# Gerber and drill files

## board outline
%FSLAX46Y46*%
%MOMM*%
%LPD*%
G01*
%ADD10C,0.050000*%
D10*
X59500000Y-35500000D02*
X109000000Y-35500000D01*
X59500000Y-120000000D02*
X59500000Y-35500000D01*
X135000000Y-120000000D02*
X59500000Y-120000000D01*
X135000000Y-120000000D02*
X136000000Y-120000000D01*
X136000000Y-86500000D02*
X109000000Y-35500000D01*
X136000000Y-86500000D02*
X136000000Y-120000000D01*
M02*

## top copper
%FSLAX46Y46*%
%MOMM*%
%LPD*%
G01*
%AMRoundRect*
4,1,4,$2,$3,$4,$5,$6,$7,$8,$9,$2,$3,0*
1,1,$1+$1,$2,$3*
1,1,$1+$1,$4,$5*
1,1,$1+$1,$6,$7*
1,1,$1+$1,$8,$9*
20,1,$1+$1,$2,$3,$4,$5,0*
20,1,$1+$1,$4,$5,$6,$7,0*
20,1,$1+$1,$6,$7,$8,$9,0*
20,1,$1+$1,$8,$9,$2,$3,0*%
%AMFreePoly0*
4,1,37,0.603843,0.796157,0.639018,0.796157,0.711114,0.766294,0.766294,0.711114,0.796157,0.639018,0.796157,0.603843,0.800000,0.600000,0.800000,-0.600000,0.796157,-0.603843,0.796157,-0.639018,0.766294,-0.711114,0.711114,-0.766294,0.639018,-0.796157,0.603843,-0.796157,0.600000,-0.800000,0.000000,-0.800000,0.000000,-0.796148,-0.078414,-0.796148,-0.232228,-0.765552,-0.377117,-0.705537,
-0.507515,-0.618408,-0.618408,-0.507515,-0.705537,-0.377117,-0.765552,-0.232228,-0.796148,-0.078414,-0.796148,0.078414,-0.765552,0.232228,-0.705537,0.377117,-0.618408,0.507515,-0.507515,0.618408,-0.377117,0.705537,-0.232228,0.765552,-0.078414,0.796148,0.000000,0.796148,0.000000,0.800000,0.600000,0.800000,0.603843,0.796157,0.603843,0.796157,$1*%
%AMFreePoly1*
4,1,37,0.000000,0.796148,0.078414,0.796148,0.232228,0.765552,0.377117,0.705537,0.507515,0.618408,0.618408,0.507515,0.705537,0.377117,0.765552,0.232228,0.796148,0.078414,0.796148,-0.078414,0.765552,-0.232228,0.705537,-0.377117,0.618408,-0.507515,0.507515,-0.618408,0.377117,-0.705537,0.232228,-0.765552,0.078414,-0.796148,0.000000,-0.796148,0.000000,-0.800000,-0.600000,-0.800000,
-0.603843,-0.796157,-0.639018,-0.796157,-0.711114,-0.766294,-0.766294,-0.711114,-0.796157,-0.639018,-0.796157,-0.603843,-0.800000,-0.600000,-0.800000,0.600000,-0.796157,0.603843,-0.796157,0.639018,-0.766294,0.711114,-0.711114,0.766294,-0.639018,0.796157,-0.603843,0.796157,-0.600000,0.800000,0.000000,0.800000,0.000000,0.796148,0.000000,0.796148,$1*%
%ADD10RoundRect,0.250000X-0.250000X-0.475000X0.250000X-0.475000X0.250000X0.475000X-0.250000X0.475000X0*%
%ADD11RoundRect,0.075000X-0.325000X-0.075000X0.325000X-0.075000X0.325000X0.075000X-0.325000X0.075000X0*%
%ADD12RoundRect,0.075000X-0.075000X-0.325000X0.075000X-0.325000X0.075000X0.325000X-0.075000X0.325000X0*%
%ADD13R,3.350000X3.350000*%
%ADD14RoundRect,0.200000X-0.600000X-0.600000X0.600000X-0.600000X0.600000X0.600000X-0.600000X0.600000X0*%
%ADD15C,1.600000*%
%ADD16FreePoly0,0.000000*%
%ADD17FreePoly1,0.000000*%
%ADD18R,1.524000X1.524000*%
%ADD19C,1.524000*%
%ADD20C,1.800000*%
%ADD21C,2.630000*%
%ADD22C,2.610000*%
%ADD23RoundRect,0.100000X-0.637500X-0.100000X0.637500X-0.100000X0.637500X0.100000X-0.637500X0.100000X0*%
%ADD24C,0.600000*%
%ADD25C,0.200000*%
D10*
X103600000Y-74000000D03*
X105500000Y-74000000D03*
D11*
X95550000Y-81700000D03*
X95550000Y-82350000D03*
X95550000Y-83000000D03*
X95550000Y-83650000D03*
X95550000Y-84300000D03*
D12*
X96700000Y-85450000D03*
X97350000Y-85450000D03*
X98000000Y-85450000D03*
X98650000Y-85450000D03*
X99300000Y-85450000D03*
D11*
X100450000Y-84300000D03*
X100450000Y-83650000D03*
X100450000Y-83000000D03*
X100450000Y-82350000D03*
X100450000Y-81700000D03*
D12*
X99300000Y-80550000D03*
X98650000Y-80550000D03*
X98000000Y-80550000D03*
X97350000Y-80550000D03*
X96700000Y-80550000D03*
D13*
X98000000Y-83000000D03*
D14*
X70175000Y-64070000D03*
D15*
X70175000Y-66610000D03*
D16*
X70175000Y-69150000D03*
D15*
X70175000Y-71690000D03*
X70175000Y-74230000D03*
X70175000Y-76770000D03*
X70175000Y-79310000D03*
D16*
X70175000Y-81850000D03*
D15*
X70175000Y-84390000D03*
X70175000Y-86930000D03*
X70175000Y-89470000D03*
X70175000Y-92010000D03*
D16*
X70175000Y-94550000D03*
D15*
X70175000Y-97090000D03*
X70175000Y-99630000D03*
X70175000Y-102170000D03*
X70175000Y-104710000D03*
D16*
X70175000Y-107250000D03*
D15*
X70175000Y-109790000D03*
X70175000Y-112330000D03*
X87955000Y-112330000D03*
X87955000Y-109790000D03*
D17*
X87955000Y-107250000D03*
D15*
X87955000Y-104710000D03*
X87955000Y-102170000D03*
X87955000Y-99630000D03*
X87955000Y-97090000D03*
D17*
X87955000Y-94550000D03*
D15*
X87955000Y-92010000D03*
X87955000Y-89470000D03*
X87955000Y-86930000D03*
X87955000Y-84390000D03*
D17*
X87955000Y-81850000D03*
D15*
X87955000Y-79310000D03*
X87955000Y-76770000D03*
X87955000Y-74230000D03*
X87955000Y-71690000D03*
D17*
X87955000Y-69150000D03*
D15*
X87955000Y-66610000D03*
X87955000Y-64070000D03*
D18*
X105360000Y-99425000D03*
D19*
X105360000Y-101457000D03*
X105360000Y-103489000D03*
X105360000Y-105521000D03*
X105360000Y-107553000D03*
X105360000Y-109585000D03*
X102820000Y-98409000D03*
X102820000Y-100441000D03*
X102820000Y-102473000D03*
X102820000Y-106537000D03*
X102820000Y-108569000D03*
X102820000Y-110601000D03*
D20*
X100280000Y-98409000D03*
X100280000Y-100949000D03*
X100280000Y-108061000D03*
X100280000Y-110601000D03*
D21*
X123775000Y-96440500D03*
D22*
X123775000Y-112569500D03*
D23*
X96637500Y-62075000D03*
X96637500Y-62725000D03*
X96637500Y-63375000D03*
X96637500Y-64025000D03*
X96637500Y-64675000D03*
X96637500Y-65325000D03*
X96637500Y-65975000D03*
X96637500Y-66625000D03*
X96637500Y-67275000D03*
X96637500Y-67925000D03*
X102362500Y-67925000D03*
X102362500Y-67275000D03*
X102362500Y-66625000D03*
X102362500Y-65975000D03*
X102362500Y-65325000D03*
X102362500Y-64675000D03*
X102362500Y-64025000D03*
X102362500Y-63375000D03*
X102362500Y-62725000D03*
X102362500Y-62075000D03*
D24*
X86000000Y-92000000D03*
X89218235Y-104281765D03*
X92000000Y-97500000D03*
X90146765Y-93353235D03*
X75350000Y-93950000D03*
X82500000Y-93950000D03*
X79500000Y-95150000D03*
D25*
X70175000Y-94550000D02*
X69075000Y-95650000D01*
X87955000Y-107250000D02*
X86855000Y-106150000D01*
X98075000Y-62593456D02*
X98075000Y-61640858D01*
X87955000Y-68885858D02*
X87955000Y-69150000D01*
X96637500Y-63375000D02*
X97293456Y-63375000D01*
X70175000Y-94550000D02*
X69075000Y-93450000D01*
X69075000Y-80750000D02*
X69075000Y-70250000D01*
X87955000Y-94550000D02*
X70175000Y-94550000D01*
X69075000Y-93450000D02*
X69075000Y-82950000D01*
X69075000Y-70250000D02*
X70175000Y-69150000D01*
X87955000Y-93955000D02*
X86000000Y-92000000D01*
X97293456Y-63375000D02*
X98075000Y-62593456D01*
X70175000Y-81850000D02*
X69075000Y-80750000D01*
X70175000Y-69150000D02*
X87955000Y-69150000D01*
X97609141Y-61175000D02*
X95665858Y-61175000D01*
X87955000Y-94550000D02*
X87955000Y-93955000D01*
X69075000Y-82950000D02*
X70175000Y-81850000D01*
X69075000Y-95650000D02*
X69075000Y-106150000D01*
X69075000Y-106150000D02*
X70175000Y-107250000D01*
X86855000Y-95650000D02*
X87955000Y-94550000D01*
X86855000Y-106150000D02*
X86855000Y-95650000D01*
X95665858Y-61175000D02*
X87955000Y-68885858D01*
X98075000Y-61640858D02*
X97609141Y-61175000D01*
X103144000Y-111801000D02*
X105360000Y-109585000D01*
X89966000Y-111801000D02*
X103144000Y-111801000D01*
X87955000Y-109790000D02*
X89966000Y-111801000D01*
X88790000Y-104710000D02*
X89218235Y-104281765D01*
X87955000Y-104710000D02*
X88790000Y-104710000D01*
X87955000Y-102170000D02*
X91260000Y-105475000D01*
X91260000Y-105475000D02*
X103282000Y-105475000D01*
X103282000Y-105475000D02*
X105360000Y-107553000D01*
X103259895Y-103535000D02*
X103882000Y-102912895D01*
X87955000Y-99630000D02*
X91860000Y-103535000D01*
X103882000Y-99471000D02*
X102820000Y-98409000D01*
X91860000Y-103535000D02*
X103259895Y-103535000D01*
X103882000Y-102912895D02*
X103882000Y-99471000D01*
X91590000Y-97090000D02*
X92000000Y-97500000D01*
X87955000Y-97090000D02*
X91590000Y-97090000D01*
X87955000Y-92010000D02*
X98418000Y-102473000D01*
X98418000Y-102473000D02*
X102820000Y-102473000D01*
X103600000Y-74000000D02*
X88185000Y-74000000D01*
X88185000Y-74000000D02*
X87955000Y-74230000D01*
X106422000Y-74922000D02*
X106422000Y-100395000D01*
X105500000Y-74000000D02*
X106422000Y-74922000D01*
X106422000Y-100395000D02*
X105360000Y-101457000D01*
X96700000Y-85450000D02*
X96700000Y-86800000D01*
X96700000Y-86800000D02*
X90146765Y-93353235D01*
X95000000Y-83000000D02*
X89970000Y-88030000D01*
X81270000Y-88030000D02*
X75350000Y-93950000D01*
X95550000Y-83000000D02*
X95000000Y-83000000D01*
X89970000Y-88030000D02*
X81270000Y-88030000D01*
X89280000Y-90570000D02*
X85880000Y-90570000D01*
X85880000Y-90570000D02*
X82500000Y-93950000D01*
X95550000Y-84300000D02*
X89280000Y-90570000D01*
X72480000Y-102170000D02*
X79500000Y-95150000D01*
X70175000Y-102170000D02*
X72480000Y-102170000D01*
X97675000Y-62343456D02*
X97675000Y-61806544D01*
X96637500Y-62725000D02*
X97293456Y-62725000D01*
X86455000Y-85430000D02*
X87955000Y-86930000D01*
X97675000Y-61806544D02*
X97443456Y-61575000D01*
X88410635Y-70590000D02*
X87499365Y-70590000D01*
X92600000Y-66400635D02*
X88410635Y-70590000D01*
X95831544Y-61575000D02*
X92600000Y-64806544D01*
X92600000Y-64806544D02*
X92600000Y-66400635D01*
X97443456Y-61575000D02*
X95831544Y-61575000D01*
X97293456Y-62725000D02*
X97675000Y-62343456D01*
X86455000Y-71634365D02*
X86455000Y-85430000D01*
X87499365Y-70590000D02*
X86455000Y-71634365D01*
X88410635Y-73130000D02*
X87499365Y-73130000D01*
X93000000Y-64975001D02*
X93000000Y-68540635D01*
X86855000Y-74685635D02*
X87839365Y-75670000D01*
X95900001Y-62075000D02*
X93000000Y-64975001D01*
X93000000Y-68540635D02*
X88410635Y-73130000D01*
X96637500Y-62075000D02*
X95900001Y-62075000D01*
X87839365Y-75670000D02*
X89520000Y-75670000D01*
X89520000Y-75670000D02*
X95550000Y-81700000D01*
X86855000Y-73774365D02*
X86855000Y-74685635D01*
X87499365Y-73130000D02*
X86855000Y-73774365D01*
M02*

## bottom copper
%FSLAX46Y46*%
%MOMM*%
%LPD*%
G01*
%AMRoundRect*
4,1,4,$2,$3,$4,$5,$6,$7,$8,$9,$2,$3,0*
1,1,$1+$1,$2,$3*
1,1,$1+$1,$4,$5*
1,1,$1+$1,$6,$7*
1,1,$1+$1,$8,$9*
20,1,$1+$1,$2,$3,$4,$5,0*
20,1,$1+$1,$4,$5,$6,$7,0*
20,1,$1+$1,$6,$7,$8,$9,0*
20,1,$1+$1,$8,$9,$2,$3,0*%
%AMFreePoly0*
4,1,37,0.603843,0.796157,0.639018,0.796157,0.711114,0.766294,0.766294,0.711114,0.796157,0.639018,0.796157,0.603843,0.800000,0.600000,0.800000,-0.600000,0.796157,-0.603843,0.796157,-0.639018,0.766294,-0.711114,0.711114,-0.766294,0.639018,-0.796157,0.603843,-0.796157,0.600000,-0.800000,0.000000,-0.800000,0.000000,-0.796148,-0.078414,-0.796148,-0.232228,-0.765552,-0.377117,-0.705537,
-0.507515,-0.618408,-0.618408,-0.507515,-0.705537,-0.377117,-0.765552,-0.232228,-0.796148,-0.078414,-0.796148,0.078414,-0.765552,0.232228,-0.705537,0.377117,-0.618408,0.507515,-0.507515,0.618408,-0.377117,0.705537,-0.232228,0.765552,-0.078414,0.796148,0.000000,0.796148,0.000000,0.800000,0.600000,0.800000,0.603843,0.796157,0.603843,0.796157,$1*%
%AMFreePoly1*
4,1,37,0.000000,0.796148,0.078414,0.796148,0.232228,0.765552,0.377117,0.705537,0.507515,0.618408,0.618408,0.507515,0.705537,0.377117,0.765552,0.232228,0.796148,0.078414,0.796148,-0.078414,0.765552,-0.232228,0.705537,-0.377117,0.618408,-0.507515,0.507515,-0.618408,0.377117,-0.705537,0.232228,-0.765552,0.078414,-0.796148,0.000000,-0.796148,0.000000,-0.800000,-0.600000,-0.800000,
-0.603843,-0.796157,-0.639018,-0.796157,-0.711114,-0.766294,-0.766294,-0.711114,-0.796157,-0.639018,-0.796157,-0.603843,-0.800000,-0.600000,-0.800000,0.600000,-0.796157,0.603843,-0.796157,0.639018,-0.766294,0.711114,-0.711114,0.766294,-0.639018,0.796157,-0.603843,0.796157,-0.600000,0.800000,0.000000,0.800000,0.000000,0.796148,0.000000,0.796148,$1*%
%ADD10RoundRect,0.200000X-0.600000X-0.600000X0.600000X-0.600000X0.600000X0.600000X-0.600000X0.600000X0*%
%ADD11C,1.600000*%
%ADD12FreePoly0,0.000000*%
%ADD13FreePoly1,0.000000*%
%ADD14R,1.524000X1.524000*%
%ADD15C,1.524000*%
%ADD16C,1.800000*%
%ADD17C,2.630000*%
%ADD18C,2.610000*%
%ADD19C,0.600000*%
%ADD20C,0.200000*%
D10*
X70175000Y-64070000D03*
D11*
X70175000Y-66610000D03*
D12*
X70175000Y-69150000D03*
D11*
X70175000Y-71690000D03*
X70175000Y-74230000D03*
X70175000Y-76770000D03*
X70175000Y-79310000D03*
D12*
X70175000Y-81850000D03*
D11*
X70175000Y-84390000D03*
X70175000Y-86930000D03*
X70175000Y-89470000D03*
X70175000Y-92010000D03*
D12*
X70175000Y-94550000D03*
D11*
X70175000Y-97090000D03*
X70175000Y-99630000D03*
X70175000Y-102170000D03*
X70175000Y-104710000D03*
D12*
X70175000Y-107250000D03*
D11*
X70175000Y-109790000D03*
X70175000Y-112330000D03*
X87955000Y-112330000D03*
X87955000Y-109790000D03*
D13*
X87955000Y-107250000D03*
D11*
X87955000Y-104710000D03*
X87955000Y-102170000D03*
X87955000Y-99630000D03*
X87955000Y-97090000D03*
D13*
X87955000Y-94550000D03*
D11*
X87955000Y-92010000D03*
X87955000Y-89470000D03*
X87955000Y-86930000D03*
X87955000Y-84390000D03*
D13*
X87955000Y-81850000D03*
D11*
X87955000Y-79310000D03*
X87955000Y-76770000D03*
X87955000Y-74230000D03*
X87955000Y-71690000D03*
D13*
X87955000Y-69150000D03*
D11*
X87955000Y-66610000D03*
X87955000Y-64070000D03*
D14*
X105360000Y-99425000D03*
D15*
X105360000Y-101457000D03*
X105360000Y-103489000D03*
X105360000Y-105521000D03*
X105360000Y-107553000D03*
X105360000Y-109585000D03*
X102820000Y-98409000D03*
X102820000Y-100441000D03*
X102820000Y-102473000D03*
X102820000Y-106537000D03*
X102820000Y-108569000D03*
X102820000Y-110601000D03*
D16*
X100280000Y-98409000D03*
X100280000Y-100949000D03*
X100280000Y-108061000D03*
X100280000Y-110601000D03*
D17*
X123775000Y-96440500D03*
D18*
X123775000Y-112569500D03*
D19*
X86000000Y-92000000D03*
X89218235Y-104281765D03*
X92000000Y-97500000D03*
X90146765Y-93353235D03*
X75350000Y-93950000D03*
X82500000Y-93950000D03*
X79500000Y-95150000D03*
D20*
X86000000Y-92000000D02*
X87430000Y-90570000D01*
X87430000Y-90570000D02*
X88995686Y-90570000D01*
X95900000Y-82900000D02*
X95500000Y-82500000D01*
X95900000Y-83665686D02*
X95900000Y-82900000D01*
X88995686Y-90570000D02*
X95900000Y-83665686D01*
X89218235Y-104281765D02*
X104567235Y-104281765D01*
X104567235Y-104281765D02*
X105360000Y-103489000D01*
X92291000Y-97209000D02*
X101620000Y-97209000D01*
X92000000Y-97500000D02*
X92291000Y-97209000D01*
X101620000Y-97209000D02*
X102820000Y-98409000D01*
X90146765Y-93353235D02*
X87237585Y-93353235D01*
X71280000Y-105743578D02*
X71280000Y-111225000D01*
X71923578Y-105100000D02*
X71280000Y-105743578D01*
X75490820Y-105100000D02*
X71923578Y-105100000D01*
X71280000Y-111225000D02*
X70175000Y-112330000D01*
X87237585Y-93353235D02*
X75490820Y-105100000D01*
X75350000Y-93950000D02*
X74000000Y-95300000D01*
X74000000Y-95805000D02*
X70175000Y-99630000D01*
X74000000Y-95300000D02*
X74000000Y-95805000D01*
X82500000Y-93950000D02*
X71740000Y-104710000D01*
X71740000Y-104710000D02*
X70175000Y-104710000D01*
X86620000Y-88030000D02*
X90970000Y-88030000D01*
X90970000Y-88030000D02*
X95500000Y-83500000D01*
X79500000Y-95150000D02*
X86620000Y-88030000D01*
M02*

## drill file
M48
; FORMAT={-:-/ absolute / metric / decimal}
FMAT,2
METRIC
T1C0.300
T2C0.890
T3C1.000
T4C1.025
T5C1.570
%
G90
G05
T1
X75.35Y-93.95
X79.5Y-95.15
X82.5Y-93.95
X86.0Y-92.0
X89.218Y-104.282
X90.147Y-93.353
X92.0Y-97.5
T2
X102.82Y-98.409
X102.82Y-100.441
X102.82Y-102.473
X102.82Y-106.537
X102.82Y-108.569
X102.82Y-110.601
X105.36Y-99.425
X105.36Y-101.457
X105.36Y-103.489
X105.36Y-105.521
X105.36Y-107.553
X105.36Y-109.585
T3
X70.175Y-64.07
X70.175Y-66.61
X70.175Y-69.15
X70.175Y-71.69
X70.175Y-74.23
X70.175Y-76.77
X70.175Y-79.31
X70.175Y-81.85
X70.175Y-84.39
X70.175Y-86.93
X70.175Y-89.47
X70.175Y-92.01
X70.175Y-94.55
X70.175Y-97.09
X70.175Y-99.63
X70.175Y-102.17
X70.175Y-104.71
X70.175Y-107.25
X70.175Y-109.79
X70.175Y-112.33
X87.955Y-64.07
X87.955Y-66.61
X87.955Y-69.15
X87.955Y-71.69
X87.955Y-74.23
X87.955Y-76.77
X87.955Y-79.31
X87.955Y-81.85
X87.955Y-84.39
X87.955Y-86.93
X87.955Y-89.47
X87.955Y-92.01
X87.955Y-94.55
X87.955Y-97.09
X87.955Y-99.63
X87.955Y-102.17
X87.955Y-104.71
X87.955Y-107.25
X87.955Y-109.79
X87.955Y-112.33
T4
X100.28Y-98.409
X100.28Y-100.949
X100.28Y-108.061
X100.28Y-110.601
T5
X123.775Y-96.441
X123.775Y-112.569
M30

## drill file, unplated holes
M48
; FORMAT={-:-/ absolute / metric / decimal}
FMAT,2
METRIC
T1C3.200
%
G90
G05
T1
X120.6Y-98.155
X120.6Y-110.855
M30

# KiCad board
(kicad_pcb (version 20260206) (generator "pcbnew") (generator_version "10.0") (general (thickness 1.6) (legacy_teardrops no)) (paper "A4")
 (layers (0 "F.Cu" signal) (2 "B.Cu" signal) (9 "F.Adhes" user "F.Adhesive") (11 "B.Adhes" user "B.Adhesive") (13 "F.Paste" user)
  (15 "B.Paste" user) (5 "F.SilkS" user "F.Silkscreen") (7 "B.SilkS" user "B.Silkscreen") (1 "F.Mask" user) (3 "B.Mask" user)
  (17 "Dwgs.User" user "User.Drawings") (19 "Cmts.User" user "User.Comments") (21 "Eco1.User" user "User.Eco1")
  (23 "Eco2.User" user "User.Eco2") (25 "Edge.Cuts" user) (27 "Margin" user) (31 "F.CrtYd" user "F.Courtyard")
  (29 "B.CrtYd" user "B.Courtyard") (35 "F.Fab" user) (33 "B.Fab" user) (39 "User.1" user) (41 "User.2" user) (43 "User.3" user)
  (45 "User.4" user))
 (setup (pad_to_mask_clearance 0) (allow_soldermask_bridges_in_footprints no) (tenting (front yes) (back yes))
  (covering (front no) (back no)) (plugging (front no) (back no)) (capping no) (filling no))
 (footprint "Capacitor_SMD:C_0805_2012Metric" (layer "F.Cu") (at 104.55 74)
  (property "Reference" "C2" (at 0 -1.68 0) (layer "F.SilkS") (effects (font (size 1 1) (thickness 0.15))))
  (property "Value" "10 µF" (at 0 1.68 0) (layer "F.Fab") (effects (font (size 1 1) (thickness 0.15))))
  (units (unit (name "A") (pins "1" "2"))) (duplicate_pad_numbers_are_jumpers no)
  (pad "1" smd roundrect (at -0.95 0) (size 1 1.45) (layers "F.Cu" "F.Mask" "F.Paste") (roundrect_rratio 0.25) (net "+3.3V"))
  (pad "2" smd roundrect (at 0.95 0) (size 1 1.45) (layers "F.Cu" "F.Mask" "F.Paste") (roundrect_rratio 0.25) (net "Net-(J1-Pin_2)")))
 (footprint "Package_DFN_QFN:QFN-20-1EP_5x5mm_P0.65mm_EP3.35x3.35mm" (layer "F.Cu") (at 98 83)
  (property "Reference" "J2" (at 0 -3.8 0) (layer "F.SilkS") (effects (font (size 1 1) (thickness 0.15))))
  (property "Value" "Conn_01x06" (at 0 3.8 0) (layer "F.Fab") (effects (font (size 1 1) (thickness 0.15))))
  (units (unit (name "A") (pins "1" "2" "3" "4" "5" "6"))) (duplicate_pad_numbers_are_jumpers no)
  (pad "" smd roundrect (at -0.84 -0.84) (size 1.35 1.35) (layers "F.Paste") (roundrect_rratio 0.185185))
  (pad "" smd roundrect (at -0.84 0.84) (size 1.35 1.35) (layers "F.Paste") (roundrect_rratio 0.185185))
  (pad "" smd roundrect (at 0.84 -0.84) (size 1.35 1.35) (layers "F.Paste") (roundrect_rratio 0.185185))
  (pad "" smd roundrect (at 0.84 0.84) (size 1.35 1.35) (layers "F.Paste") (roundrect_rratio 0.185185))
  (pad "1" smd roundrect (at -2.45 -1.3) (size 0.8 0.3) (layers "F.Cu" "F.Mask" "F.Paste") (roundrect_rratio 0.25) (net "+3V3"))
  (pad "2" smd roundrect (at -2.45 -0.65) (size 0.8 0.3) (layers "F.Cu" "F.Mask" "F.Paste") (roundrect_rratio 0.25) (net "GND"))
  (pad "3" smd roundrect (at -2.45 0) (size 0.8 0.3) (layers "F.Cu" "F.Mask" "F.Paste") (roundrect_rratio 0.25) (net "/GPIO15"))
  (pad "4" smd roundrect (at -2.45 0.65) (size 0.8 0.3) (layers "F.Cu" "F.Mask" "F.Paste") (roundrect_rratio 0.25) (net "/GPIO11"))
  (pad "5" smd roundrect (at -2.45 1.3) (size 0.8 0.3) (layers "F.Cu" "F.Mask" "F.Paste") (roundrect_rratio 0.25) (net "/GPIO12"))
  (pad "6" smd roundrect (at -1.3 2.45) (size 0.3 0.8) (layers "F.Cu" "F.Mask" "F.Paste") (roundrect_rratio 0.25) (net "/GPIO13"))
  (pad "7" smd roundrect (at -0.65 2.45) (size 0.3 0.8) (layers "F.Cu" "F.Mask" "F.Paste") (roundrect_rratio 0.25))
  (pad "8" smd roundrect (at 0 2.45) (size 0.3 0.8) (layers "F.Cu" "F.Mask" "F.Paste") (roundrect_rratio 0.25))
  (pad "9" smd roundrect (at 0.65 2.45) (size 0.3 0.8) (layers "F.Cu" "F.Mask" "F.Paste") (roundrect_rratio 0.25))
  (pad "10" smd roundrect (at 1.3 2.45) (size 0.3 0.8) (layers "F.Cu" "F.Mask" "F.Paste") (roundrect_rratio 0.25))
  (pad "11" smd roundrect (at 2.45 1.3) (size 0.8 0.3) (layers "F.Cu" "F.Mask" "F.Paste") (roundrect_rratio 0.25))
  (pad "12" smd roundrect (at 2.45 0.65) (size 0.8 0.3) (layers "F.Cu" "F.Mask" "F.Paste") (roundrect_rratio 0.25))
  (pad "13" smd roundrect (at 2.45 0) (size 0.8 0.3) (layers "F.Cu" "F.Mask" "F.Paste") (roundrect_rratio 0.25))
  (pad "14" smd roundrect (at 2.45 -0.65) (size 0.8 0.3) (layers "F.Cu" "F.Mask" "F.Paste") (roundrect_rratio 0.25))
  (pad "15" smd roundrect (at 2.45 -1.3) (size 0.8 0.3) (layers "F.Cu" "F.Mask" "F.Paste") (roundrect_rratio 0.25))
  (pad "16" smd roundrect (at 1.3 -2.45) (size 0.3 0.8) (layers "F.Cu" "F.Mask" "F.Paste") (roundrect_rratio 0.25))
  (pad "17" smd roundrect (at 0.65 -2.45) (size 0.3 0.8) (layers "F.Cu" "F.Mask" "F.Paste") (roundrect_rratio 0.25))
  (pad "18" smd roundrect (at 0 -2.45) (size 0.3 0.8) (layers "F.Cu" "F.Mask" "F.Paste") (roundrect_rratio 0.25))
  (pad "19" smd roundrect (at -0.65 -2.45) (size 0.3 0.8) (layers "F.Cu" "F.Mask" "F.Paste") (roundrect_rratio 0.25))
  (pad "20" smd roundrect (at -1.3 -2.45) (size 0.3 0.8) (layers "F.Cu" "F.Mask" "F.Paste") (roundrect_rratio 0.25))
  (pad "21" smd rect (at 0 0) (size 3.35 3.35) (layers "F.Cu" "F.Mask") (zone_connect 2)))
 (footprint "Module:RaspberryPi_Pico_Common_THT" (layer "F.Cu") (at 70.175 64.07)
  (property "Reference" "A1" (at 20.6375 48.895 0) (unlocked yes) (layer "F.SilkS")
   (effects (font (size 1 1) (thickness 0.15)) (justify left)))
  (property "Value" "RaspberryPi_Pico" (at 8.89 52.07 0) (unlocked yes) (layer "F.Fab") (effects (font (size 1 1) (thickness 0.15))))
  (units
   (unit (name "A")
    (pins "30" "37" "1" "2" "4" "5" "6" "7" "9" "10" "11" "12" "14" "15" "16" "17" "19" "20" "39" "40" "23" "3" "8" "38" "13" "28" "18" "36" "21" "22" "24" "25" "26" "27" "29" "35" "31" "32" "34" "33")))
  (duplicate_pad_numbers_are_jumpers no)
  (pad "1" thru_hole roundrect (at 0 0) (size 1.6 1.6) (drill 1) (layers "*.Cu" "*.Mask") (remove_unused_layers no) (roundrect_rratio 0.125)
   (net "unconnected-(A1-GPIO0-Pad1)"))
  (pad "2" thru_hole circle (at 0 2.54) (size 1.6 1.6) (drill 1) (layers "*.Cu" "*.Mask") (remove_unused_layers no)
   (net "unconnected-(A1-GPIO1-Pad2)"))
  (pad "3" thru_hole custom (at 0 5.08) (size 1.6 1.6) (drill 1) (layers "*.Cu" "*.Mask") (remove_unused_layers no) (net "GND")
   (options (clearance outline) (anchor circle)) (primitives))
  (pad "4" thru_hole circle (at 0 7.62) (size 1.6 1.6) (drill 1) (layers "*.Cu" "*.Mask") (remove_unused_layers no)
   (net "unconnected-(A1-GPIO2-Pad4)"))
  (pad "5" thru_hole circle (at 0 10.16) (size 1.6 1.6) (drill 1) (layers "*.Cu" "*.Mask") (remove_unused_layers no)
   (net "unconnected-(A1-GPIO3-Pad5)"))
  (pad "6" thru_hole circle (at 0 12.7) (size 1.6 1.6) (drill 1) (layers "*.Cu" "*.Mask") (remove_unused_layers no)
   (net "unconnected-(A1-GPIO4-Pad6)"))
  (pad "7" thru_hole circle (at 0 15.24) (size 1.6 1.6) (drill 1) (layers "*.Cu" "*.Mask") (remove_unused_layers no)
   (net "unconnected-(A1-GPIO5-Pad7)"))
  (pad "8" thru_hole custom (at 0 17.78) (size 1.6 1.6) (drill 1) (layers "*.Cu" "*.Mask") (remove_unused_layers no) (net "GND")
   (options (clearance outline) (anchor circle)) (primitives))
  (pad "9" thru_hole circle (at 0 20.32) (size 1.6 1.6) (drill 1) (layers "*.Cu" "*.Mask") (remove_unused_layers no)
   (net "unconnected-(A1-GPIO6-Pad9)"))
  (pad "10" thru_hole circle (at 0 22.86) (size 1.6 1.6) (drill 1) (layers "*.Cu" "*.Mask") (remove_unused_layers no)
   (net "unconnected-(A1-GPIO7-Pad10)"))
  (pad "11" thru_hole circle (at 0 25.4) (size 1.6 1.6) (drill 1) (layers "*.Cu" "*.Mask") (remove_unused_layers no)
   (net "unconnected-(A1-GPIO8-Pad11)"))
  (pad "12" thru_hole circle (at 0 27.94) (size 1.6 1.6) (drill 1) (layers "*.Cu" "*.Mask") (remove_unused_layers no)
   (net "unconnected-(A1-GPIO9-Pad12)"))
  (pad "13" thru_hole custom (at 0 30.48) (size 1.6 1.6) (drill 1) (layers "*.Cu" "*.Mask") (remove_unused_layers no) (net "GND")
   (options (clearance outline) (anchor circle)) (primitives))
  (pad "14" thru_hole circle (at 0 33.02) (size 1.6 1.6) (drill 1) (layers "*.Cu" "*.Mask") (remove_unused_layers no)
   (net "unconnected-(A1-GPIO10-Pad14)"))
  (pad "15" thru_hole circle (at 0 35.56) (size 1.6 1.6) (drill 1) (layers "*.Cu" "*.Mask") (remove_unused_layers no) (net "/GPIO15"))
  (pad "16" thru_hole circle (at 0 38.1) (size 1.6 1.6) (drill 1) (layers "*.Cu" "*.Mask") (remove_unused_layers no) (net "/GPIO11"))
  (pad "17" thru_hole circle (at 0 40.64) (size 1.6 1.6) (drill 1) (layers "*.Cu" "*.Mask") (remove_unused_layers no) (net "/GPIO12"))
  (pad "18" thru_hole custom (at 0 43.18) (size 1.6 1.6) (drill 1) (layers "*.Cu" "*.Mask") (remove_unused_layers no) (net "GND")
   (options (clearance outline) (anchor circle)) (primitives))
  (pad "19" thru_hole circle (at 0 45.72) (size 1.6 1.6) (drill 1) (layers "*.Cu" "*.Mask") (remove_unused_layers no)
   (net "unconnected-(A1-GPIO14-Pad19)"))
  (pad "20" thru_hole circle (at 0 48.26) (size 1.6 1.6) (drill 1) (layers "*.Cu" "*.Mask") (remove_unused_layers no) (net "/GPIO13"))
  (pad "21" thru_hole circle (at 17.78 48.26) (size 1.6 1.6) (drill 1) (layers "*.Cu" "*.Mask") (remove_unused_layers no)
   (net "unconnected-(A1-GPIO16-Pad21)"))
  (pad "22" thru_hole circle (at 17.78 45.72) (size 1.6 1.6) (drill 1) (layers "*.Cu" "*.Mask") (remove_unused_layers no) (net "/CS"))
  (pad "23" thru_hole custom (at 17.78 43.18) (size 1.6 1.6) (drill 1) (layers "*.Cu" "*.Mask") (remove_unused_layers no) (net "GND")
   (options (clearance outline) (anchor circle)) (primitives))
  (pad "24" thru_hole circle (at 17.78 40.64) (size 1.6 1.6) (drill 1) (layers "*.Cu" "*.Mask") (remove_unused_layers no) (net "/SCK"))
  (pad "25" thru_hole circle (at 17.78 38.1) (size 1.6 1.6) (drill 1) (layers "*.Cu" "*.Mask") (remove_unused_layers no) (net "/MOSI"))
  (pad "26" thru_hole circle (at 17.78 35.56) (size 1.6 1.6) (drill 1) (layers "*.Cu" "*.Mask") (remove_unused_layers no) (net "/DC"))
  (pad "27" thru_hole circle (at 17.78 33.02) (size 1.6 1.6) (drill 1) (layers "*.Cu" "*.Mask") (remove_unused_layers no) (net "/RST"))
  (pad "28" thru_hole custom (at 17.78 30.48) (size 1.6 1.6) (drill 1) (layers "*.Cu" "*.Mask") (remove_unused_layers no) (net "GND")
   (options (clearance outline) (anchor circle)) (primitives))
  (pad "29" thru_hole circle (at 17.78 27.94) (size 1.6 1.6) (drill 1) (layers "*.Cu" "*.Mask") (remove_unused_layers no) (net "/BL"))
  (pad "30" thru_hole circle (at 17.78 25.4) (size 1.6 1.6) (drill 1) (layers "*.Cu" "*.Mask") (remove_unused_layers no)
   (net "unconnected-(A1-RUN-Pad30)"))
  (pad "31" thru_hole circle (at 17.78 22.86) (size 1.6 1.6) (drill 1) (layers "*.Cu" "*.Mask") (remove_unused_layers no) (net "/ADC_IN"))
  (pad "32" thru_hole circle (at 17.78 20.32) (size 1.6 1.6) (drill 1) (layers "*.Cu" "*.Mask") (remove_unused_layers no)
   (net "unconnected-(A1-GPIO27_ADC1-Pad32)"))
  (pad "33" thru_hole custom (at 17.78 17.78) (size 1.6 1.6) (drill 1) (layers "*.Cu" "*.Mask") (remove_unused_layers no)
   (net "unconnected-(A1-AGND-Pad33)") (options (clearance outline) (anchor circle)) (primitives))
  (pad "34" thru_hole circle (at 17.78 15.24) (size 1.6 1.6) (drill 1) (layers "*.Cu" "*.Mask") (remove_unused_layers no)
   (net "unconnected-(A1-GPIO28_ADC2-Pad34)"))
  (pad "35" thru_hole circle (at 17.78 12.7) (size 1.6 1.6) (drill 1) (layers "*.Cu" "*.Mask") (remove_unused_layers no)
   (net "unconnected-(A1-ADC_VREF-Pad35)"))
  (pad "36" thru_hole circle (at 17.78 10.16) (size 1.6 1.6) (drill 1) (layers "*.Cu" "*.Mask") (remove_unused_layers no) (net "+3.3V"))
  (pad "37" thru_hole circle (at 17.78 7.62) (size 1.6 1.6) (drill 1) (layers "*.Cu" "*.Mask") (remove_unused_layers no)
   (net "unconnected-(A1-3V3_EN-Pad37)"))
  (pad "38" thru_hole custom (at 17.78 5.08) (size 1.6 1.6) (drill 1) (layers "*.Cu" "*.Mask") (remove_unused_layers no) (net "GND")
   (options (clearance outline) (anchor circle)) (primitives))
  (pad "39" thru_hole circle (at 17.78 2.54) (size 1.6 1.6) (drill 1) (layers "*.Cu" "*.Mask") (remove_unused_layers no)
   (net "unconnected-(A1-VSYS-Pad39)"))
  (pad "40" thru_hole circle (at 17.78 0) (size 1.6 1.6) (drill 1) (layers "*.Cu" "*.Mask") (remove_unused_layers no)
   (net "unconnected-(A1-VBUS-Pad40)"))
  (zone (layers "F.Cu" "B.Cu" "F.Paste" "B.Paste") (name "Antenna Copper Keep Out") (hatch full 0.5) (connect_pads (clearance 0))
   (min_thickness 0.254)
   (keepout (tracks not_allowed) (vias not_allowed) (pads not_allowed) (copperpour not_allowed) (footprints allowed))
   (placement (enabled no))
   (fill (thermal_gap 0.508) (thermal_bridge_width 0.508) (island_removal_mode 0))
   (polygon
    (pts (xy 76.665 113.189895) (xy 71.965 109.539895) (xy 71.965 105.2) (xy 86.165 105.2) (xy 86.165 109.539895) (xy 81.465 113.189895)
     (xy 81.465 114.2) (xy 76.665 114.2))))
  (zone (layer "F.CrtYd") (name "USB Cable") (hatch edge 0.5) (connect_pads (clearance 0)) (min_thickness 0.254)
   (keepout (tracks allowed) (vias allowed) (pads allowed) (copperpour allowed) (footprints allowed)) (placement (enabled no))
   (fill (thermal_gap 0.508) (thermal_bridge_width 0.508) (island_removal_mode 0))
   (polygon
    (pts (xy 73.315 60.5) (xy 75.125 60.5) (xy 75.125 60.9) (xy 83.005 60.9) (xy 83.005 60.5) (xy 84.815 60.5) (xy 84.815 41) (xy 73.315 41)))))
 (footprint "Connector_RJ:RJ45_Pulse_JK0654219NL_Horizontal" (layer "F.Cu") (at 105.36 99.425)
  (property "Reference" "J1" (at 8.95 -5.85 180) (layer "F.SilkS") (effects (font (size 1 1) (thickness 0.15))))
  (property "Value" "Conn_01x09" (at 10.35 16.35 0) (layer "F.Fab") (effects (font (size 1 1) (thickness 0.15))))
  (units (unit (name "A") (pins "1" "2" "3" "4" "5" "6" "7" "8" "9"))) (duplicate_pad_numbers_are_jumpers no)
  (pad "" np_thru_hole circle (at 15.24 -1.27 180) (size 3.2 3.2) (drill 3.2) (layers "*.Cu" "*.Mask"))
  (pad "" np_thru_hole circle (at 15.24 11.43 180) (size 3.2 3.2) (drill 3.2) (layers "*.Cu" "*.Mask"))
  (pad "1" thru_hole rect (at 0 0 180) (size 1.524 1.524) (drill 0.89) (layers "*.Cu" "*.Mask") (remove_unused_layers no)
   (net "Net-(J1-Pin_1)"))
  (pad "2" thru_hole circle (at 0 2.032 180) (size 1.524 1.524) (drill 0.89) (layers "*.Cu" "*.Mask") (remove_unused_layers no)
   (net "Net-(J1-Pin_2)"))
  (pad "3" thru_hole circle (at 0 4.064 180) (size 1.524 1.524) (drill 0.89) (layers "*.Cu" "*.Mask") (remove_unused_layers no) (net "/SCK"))
  (pad "4" thru_hole circle (at 0 6.096 180) (size 1.524 1.524) (drill 0.89) (layers "*.Cu" "*.Mask") (remove_unused_layers no)
   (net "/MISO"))
  (pad "5" thru_hole circle (at 0 8.128 180) (size 1.524 1.524) (drill 0.89) (layers "*.Cu" "*.Mask") (remove_unused_layers no)
   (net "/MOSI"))
  (pad "6" thru_hole circle (at 0 10.16 180) (size 1.524 1.524) (drill 0.89) (layers "*.Cu" "*.Mask") (remove_unused_layers no) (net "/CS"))
  (pad "7" thru_hole circle (at -2.54 -1.016 180) (size 1.524 1.524) (drill 0.89) (layers "*.Cu" "*.Mask") (remove_unused_layers no)
   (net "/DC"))
  (pad "8" thru_hole circle (at -2.54 1.016 180) (size 1.524 1.524) (drill 0.89) (layers "*.Cu" "*.Mask") (remove_unused_layers no)
   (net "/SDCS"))
  (pad "9" thru_hole circle (at -2.54 3.048 180) (size 1.524 1.524) (drill 0.89) (layers "*.Cu" "*.Mask") (remove_unused_layers no)
   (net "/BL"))
  (pad "10" thru_hole circle (at -2.54 7.112 180) (size 1.524 1.524) (drill 0.89) (layers "*.Cu" "*.Mask") (remove_unused_layers no))
  (pad "11" thru_hole circle (at -2.54 9.144 180) (size 1.524 1.524) (drill 0.89) (layers "*.Cu" "*.Mask") (remove_unused_layers no))
  (pad "12" thru_hole circle (at -2.54 11.176 180) (size 1.524 1.524) (drill 0.89) (layers "*.Cu" "*.Mask") (remove_unused_layers no))
  (pad "13" thru_hole circle (at -5.08 -1.016 180) (size 1.8 1.8) (drill 1.025) (layers "*.Cu" "*.Mask") (remove_unused_layers no))
  (pad "14" thru_hole circle (at -5.08 1.524 180) (size 1.8 1.8) (drill 1.025) (layers "*.Cu" "*.Mask") (remove_unused_layers no))
  (pad "15" thru_hole circle (at -5.08 8.636 180) (size 1.8 1.8) (drill 1.025) (layers "*.Cu" "*.Mask") (remove_unused_layers no))
  (pad "16" thru_hole circle (at -5.08 11.176 180) (size 1.8 1.8) (drill 1.025) (layers "*.Cu" "*.Mask") (remove_unused_layers no))
  (pad "SH" thru_hole circle (at 18.415 -2.9845 180) (size 2.63 2.63) (drill 1.57) (layers "*.Cu" "*.Mask") (remove_unused_layers no))
  (pad "SH" thru_hole circle (at 18.415 13.1445 180) (size 2.61 2.61) (drill 1.57) (layers "*.Cu" "*.Mask") (remove_unused_layers no)))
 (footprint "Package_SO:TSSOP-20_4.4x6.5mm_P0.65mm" (layer "F.Cu") (at 99.5 65)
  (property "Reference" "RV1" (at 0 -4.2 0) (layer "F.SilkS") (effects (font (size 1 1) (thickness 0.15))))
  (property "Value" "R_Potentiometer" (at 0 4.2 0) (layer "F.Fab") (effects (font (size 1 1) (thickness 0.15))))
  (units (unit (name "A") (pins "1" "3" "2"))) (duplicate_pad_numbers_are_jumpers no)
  (pad "1" smd roundrect (at -2.8625 -2.925) (size 1.475 0.4) (layers "F.Cu" "F.Mask" "F.Paste") (roundrect_rratio 0.25) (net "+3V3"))
  (pad "2" smd roundrect (at -2.8625 -2.275) (size 1.475 0.4) (layers "F.Cu" "F.Mask" "F.Paste") (roundrect_rratio 0.25) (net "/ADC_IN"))
  (pad "3" smd roundrect (at -2.8625 -1.625) (size 1.475 0.4) (layers "F.Cu" "F.Mask" "F.Paste") (roundrect_rratio 0.25) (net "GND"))
  (pad "4" smd roundrect (at -2.8625 -0.975) (size 1.475 0.4) (layers "F.Cu" "F.Mask" "F.Paste") (roundrect_rratio 0.25))
  (pad "5" smd roundrect (at -2.8625 -0.325) (size 1.475 0.4) (layers "F.Cu" "F.Mask" "F.Paste") (roundrect_rratio 0.25))
  (pad "6" smd roundrect (at -2.8625 0.325) (size 1.475 0.4) (layers "F.Cu" "F.Mask" "F.Paste") (roundrect_rratio 0.25))
  (pad "7" smd roundrect (at -2.8625 0.975) (size 1.475 0.4) (layers "F.Cu" "F.Mask" "F.Paste") (roundrect_rratio 0.25))
  (pad "8" smd roundrect (at -2.8625 1.625) (size 1.475 0.4) (layers "F.Cu" "F.Mask" "F.Paste") (roundrect_rratio 0.25))
  (pad "9" smd roundrect (at -2.8625 2.275) (size 1.475 0.4) (layers "F.Cu" "F.Mask" "F.Paste") (roundrect_rratio 0.25))
  (pad "10" smd roundrect (at -2.8625 2.925) (size 1.475 0.4) (layers "F.Cu" "F.Mask" "F.Paste") (roundrect_rratio 0.25))
  (pad "11" smd roundrect (at 2.8625 2.925) (size 1.475 0.4) (layers "F.Cu" "F.Mask" "F.Paste") (roundrect_rratio 0.25))
  (pad "12" smd roundrect (at 2.8625 2.275) (size 1.475 0.4) (layers "F.Cu" "F.Mask" "F.Paste") (roundrect_rratio 0.25))
  (pad "13" smd roundrect (at 2.8625 1.625) (size 1.475 0.4) (layers "F.Cu" "F.Mask" "F.Paste") (roundrect_rratio 0.25))
  (pad "14" smd roundrect (at 2.8625 0.975) (size 1.475 0.4) (layers "F.Cu" "F.Mask" "F.Paste") (roundrect_rratio 0.25))
  (pad "15" smd roundrect (at 2.8625 0.325) (size 1.475 0.4) (layers "F.Cu" "F.Mask" "F.Paste") (roundrect_rratio 0.25))
  (pad "16" smd roundrect (at 2.8625 -0.325) (size 1.475 0.4) (layers "F.Cu" "F.Mask" "F.Paste") (roundrect_rratio 0.25))
  (pad "17" smd roundrect (at 2.8625 -0.975) (size 1.475 0.4) (layers "F.Cu" "F.Mask" "F.Paste") (roundrect_rratio 0.25))
  (pad "18" smd roundrect (at 2.8625 -1.625) (size 1.475 0.4) (layers "F.Cu" "F.Mask" "F.Paste") (roundrect_rratio 0.25))
  (pad "19" smd roundrect (at 2.8625 -2.275) (size 1.475 0.4) (layers "F.Cu" "F.Mask" "F.Paste") (roundrect_rratio 0.25))
  (pad "20" smd roundrect (at 2.8625 -2.925) (size 1.475 0.4) (layers "F.Cu" "F.Mask" "F.Paste") (roundrect_rratio 0.25)))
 (gr_line (start 59.5 35.5) (end 109 35.5) (stroke (width 0.05) (type default)) (layer "Edge.Cuts"))
 (gr_line (start 59.5 120) (end 59.5 35.5) (stroke (width 0.05) (type default)) (layer "Edge.Cuts"))
 (gr_line (start 135 120) (end 59.5 120) (stroke (width 0.05) (type default)) (layer "Edge.Cuts"))
 (gr_line (start 135 120) (end 136 120) (stroke (width 0.05) (type default)) (layer "Edge.Cuts"))
 (gr_line (start 136 86.5) (end 109 35.5) (stroke (width 0.05) (type default)) (layer "Edge.Cuts"))
 (gr_line (start 136 86.5) (end 136 120) (stroke (width 0.05) (type default)) (layer "Edge.Cuts"))
 (segment (start 103.6 74) (end 88.185 74) (width 0.2) (layer "F.Cu") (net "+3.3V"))
 (segment (start 88.185 74) (end 87.955 74.23) (width 0.2) (layer "F.Cu") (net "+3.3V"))
 (segment (start 106.422 74.922) (end 106.422 100.395) (width 0.2) (layer "F.Cu") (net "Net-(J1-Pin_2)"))
 (segment (start 105.5 74) (end 106.422 74.922) (width 0.2) (layer "F.Cu") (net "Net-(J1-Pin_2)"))
 (segment (start 106.422 100.395) (end 105.36 101.457) (width 0.2) (layer "F.Cu") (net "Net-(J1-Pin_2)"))
 (segment (start 88.410635 73.13) (end 87.499365 73.13) (width 0.2) (layer "F.Cu") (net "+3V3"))
 (segment (start 93 64.975001) (end 93 68.540635) (width 0.2) (layer "F.Cu") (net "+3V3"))
 (segment (start 86.855 74.685635) (end 87.839365 75.67) (width 0.2) (layer "F.Cu") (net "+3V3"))
 (segment (start 95.900001 62.075) (end 93 64.975001) (width 0.2) (layer "F.Cu") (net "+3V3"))
 (segment (start 93 68.540635) (end 88.410635 73.13) (width 0.2) (layer "F.Cu") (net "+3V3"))
 (segment (start 96.6375 62.075) (end 95.900001 62.075) (width 0.2) (layer "F.Cu") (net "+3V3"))
 (segment (start 87.839365 75.67) (end 89.52 75.67) (width 0.2) (layer "F.Cu") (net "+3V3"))
 (segment (start 89.52 75.67) (end 95.55 81.7) (width 0.2) (layer "F.Cu") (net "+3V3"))
 (segment (start 86.855 73.774365) (end 86.855 74.685635) (width 0.2) (layer "F.Cu") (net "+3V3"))
 (segment (start 87.499365 73.13) (end 86.855 73.774365) (width 0.2) (layer "F.Cu") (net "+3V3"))
 (segment (start 70.175 94.55) (end 69.075 95.65) (width 0.2) (layer "F.Cu") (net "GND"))
 (segment (start 87.955 107.25) (end 86.855 106.15) (width 0.2) (layer "F.Cu") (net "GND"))
 (segment (start 98.075 62.593456) (end 98.075 61.640858) (width 0.2) (layer "F.Cu") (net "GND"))
 (segment (start 87.955 68.885858) (end 87.955 69.15) (width 0.2) (layer "F.Cu") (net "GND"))
 (segment (start 96.6375 63.375) (end 97.293456 63.375) (width 0.2) (layer "F.Cu") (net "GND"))
 (segment (start 70.175 94.55) (end 69.075 93.45) (width 0.2) (layer "F.Cu") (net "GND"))
 (segment (start 69.075 80.75) (end 69.075 70.25) (width 0.2) (layer "F.Cu") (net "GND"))
 (segment (start 87.955 94.55) (end 70.175 94.55) (width 0.2) (layer "F.Cu") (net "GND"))
 (segment (start 69.075 93.45) (end 69.075 82.95) (width 0.2) (layer "F.Cu") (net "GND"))
 (segment (start 69.075 70.25) (end 70.175 69.15) (width 0.2) (layer "F.Cu") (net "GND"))
 (segment (start 87.955 93.955) (end 86 92) (width 0.2) (layer "F.Cu") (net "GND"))
 (segment (start 97.293456 63.375) (end 98.075 62.593456) (width 0.2) (layer "F.Cu") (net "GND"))
 (segment (start 70.175 81.85) (end 69.075 80.75) (width 0.2) (layer "F.Cu") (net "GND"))
 (segment (start 70.175 69.15) (end 87.955 69.15) (width 0.2) (layer "F.Cu") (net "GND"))
 (segment (start 97.609141 61.175) (end 95.665858 61.175) (width 0.2) (layer "F.Cu") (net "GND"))
 (segment (start 87.955 94.55) (end 87.955 93.955) (width 0.2) (layer "F.Cu") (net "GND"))
 (segment (start 69.075 82.95) (end 70.175 81.85) (width 0.2) (layer "F.Cu") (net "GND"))
 (segment (start 69.075 95.65) (end 69.075 106.15) (width 0.2) (layer "F.Cu") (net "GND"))
 (segment (start 69.075 106.15) (end 70.175 107.25) (width 0.2) (layer "F.Cu") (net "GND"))
 (segment (start 86.855 95.65) (end 87.955 94.55) (width 0.2) (layer "F.Cu") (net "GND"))
 (segment (start 86.855 106.15) (end 86.855 95.65) (width 0.2) (layer "F.Cu") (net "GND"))
 (segment (start 95.665858 61.175) (end 87.955 68.885858) (width 0.2) (layer "F.Cu") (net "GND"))
 (segment (start 98.075 61.640858) (end 97.609141 61.175) (width 0.2) (layer "F.Cu") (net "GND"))
 (via (at 86 92) (size 0.6) (drill 0.3) (layers "F.Cu" "B.Cu") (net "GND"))
 (segment (start 86 92) (end 87.43 90.57) (width 0.2) (layer "B.Cu") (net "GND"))
 (segment (start 87.43 90.57) (end 88.995686 90.57) (width 0.2) (layer "B.Cu") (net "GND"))
 (segment (start 95.9 82.9) (end 95.5 82.5) (width 0.2) (layer "B.Cu") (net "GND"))
 (segment (start 95.9 83.665686) (end 95.9 82.9) (width 0.2) (layer "B.Cu") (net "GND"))
 (segment (start 88.995686 90.57) (end 95.9 83.665686) (width 0.2) (layer "B.Cu") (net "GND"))
 (segment (start 95 83) (end 89.97 88.03) (width 0.2) (layer "F.Cu") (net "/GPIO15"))
 (segment (start 81.27 88.03) (end 75.35 93.95) (width 0.2) (layer "F.Cu") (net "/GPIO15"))
 (segment (start 95.55 83) (end 95 83) (width 0.2) (layer "F.Cu") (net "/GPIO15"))
 (segment (start 89.97 88.03) (end 81.27 88.03) (width 0.2) (layer "F.Cu") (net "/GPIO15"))
 (via (at 75.35 93.95) (size 0.6) (drill 0.3) (layers "F.Cu" "B.Cu") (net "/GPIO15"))
 (segment (start 75.35 93.95) (end 74 95.3) (width 0.2) (layer "B.Cu") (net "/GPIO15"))
 (segment (start 74 95.805) (end 70.175 99.63) (width 0.2) (layer "B.Cu") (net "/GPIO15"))
 (segment (start 74 95.3) (end 74 95.805) (width 0.2) (layer "B.Cu") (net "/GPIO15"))
 (segment (start 72.48 102.17) (end 79.5 95.15) (width 0.2) (layer "F.Cu") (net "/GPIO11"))
 (segment (start 70.175 102.17) (end 72.48 102.17) (width 0.2) (layer "F.Cu") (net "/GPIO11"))
 (via (at 79.5 95.15) (size 0.6) (drill 0.3) (layers "F.Cu" "B.Cu") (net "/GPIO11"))
 (segment (start 86.62 88.03) (end 90.97 88.03) (width 0.2) (layer "B.Cu") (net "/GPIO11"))
 (segment (start 90.97 88.03) (end 95.5 83.5) (width 0.2) (layer "B.Cu") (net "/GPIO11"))
 (segment (start 79.5 95.15) (end 86.62 88.03) (width 0.2) (layer "B.Cu") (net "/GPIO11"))
 (segment (start 89.28 90.57) (end 85.88 90.57) (width 0.2) (layer "F.Cu") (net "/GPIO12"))
 (segment (start 85.88 90.57) (end 82.5 93.95) (width 0.2) (layer "F.Cu") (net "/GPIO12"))
 (segment (start 95.55 84.3) (end 89.28 90.57) (width 0.2) (layer "F.Cu") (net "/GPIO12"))
 (via (at 82.5 93.95) (size 0.6) (drill 0.3) (layers "F.Cu" "B.Cu") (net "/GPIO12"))
 (segment (start 82.5 93.95) (end 71.74 104.71) (width 0.2) (layer "B.Cu") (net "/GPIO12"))
 (segment (start 71.74 104.71) (end 70.175 104.71) (width 0.2) (layer "B.Cu") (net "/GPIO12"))
 (segment (start 96.7 85.45) (end 96.7 86.8) (width 0.2) (layer "F.Cu") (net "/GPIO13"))
 (segment (start 96.7 86.8) (end 90.146765 93.353235) (width 0.2) (layer "F.Cu") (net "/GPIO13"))
 (via (at 90.146765 93.353235) (size 0.6) (drill 0.3) (layers "F.Cu" "B.Cu") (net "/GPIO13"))
 (segment (start 90.146765 93.353235) (end 87.237585 93.353235) (width 0.2) (layer "B.Cu") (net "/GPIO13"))
 (segment (start 71.28 105.743578) (end 71.28 111.225) (width 0.2) (layer "B.Cu") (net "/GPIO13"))
 (segment (start 71.923578 105.1) (end 71.28 105.743578) (width 0.2) (layer "B.Cu") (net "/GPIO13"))
 (segment (start 75.49082 105.1) (end 71.923578 105.1) (width 0.2) (layer "B.Cu") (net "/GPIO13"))
 (segment (start 71.28 111.225) (end 70.175 112.33) (width 0.2) (layer "B.Cu") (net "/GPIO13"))
 (segment (start 87.237585 93.353235) (end 75.49082 105.1) (width 0.2) (layer "B.Cu") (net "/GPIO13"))
 (segment (start 103.144 111.801) (end 105.36 109.585) (width 0.2) (layer "F.Cu") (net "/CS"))
 (segment (start 89.966 111.801) (end 103.144 111.801) (width 0.2) (layer "F.Cu") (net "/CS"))
 (segment (start 87.955 109.79) (end 89.966 111.801) (width 0.2) (layer "F.Cu") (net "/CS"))
 (segment (start 88.79 104.71) (end 89.218235 104.281765) (width 0.2) (layer "F.Cu") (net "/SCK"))
 (segment (start 87.955 104.71) (end 88.79 104.71) (width 0.2) (layer "F.Cu") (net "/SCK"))
 (via (at 89.218235 104.281765) (size 0.6) (drill 0.3) (layers "F.Cu" "B.Cu") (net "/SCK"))
 (segment (start 89.218235 104.281765) (end 104.567235 104.281765) (width 0.2) (layer "B.Cu") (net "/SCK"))
 (segment (start 104.567235 104.281765) (end 105.36 103.489) (width 0.2) (layer "B.Cu") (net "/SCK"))
 (segment (start 87.955 102.17) (end 91.26 105.475) (width 0.2) (layer "F.Cu") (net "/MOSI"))
 (segment (start 91.26 105.475) (end 103.282 105.475) (width 0.2) (layer "F.Cu") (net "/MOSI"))
 (segment (start 103.282 105.475) (end 105.36 107.553) (width 0.2) (layer "F.Cu") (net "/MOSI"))
 (segment (start 103.259895 103.535) (end 103.882 102.912895) (width 0.2) (layer "F.Cu") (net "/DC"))
 (segment (start 87.955 99.63) (end 91.86 103.535) (width 0.2) (layer "F.Cu") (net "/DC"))
 (segment (start 103.882 99.471) (end 102.82 98.409) (width 0.2) (layer "F.Cu") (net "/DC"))
 (segment (start 91.86 103.535) (end 103.259895 103.535) (width 0.2) (layer "F.Cu") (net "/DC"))
 (segment (start 103.882 102.912895) (end 103.882 99.471) (width 0.2) (layer "F.Cu") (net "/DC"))
 (segment (start 91.59 97.09) (end 92 97.5) (width 0.2) (layer "F.Cu") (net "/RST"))
 (segment (start 87.955 97.09) (end 91.59 97.09) (width 0.2) (layer "F.Cu") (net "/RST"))
 (via (at 92 97.5) (size 0.6) (drill 0.3) (layers "F.Cu" "B.Cu") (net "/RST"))
 (segment (start 92.291 97.209) (end 101.62 97.209) (width 0.2) (layer "B.Cu") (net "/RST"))
 (segment (start 92 97.5) (end 92.291 97.209) (width 0.2) (layer "B.Cu") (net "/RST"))
 (segment (start 101.62 97.209) (end 102.82 98.409) (width 0.2) (layer "B.Cu") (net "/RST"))
 (segment (start 87.955 92.01) (end 98.418 102.473) (width 0.2) (layer "F.Cu") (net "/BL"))
 (segment (start 98.418 102.473) (end 102.82 102.473) (width 0.2) (layer "F.Cu") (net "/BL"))
 (segment (start 97.675 62.343456) (end 97.675 61.806544) (width 0.2) (layer "F.Cu") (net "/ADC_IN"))
 (segment (start 96.6375 62.725) (end 97.293456 62.725) (width 0.2) (layer "F.Cu") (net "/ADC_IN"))
 (segment (start 86.455 85.43) (end 87.955 86.93) (width 0.2) (layer "F.Cu") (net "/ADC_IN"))
 (segment (start 97.675 61.806544) (end 97.443456 61.575) (width 0.2) (layer "F.Cu") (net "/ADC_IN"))
 (segment (start 88.410635 70.59) (end 87.499365 70.59) (width 0.2) (layer "F.Cu") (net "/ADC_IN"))
 (segment (start 92.6 66.400635) (end 88.410635 70.59) (width 0.2) (layer "F.Cu") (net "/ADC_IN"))
 (segment (start 95.831544 61.575) (end 92.6 64.806544) (width 0.2) (layer "F.Cu") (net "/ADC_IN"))
 (segment (start 92.6 64.806544) (end 92.6 66.400635) (width 0.2) (layer "F.Cu") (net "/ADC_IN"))
 (segment (start 97.443456 61.575) (end 95.831544 61.575) (width 0.2) (layer "F.Cu") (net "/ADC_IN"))
 (segment (start 97.293456 62.725) (end 97.675 62.343456) (width 0.2) (layer "F.Cu") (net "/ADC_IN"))
 (segment (start 86.455 71.634365) (end 86.455 85.43) (width 0.2) (layer "F.Cu") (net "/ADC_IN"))
 (segment (start 87.499365 70.59) (end 86.455 71.634365) (width 0.2) (layer "F.Cu") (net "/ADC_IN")))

